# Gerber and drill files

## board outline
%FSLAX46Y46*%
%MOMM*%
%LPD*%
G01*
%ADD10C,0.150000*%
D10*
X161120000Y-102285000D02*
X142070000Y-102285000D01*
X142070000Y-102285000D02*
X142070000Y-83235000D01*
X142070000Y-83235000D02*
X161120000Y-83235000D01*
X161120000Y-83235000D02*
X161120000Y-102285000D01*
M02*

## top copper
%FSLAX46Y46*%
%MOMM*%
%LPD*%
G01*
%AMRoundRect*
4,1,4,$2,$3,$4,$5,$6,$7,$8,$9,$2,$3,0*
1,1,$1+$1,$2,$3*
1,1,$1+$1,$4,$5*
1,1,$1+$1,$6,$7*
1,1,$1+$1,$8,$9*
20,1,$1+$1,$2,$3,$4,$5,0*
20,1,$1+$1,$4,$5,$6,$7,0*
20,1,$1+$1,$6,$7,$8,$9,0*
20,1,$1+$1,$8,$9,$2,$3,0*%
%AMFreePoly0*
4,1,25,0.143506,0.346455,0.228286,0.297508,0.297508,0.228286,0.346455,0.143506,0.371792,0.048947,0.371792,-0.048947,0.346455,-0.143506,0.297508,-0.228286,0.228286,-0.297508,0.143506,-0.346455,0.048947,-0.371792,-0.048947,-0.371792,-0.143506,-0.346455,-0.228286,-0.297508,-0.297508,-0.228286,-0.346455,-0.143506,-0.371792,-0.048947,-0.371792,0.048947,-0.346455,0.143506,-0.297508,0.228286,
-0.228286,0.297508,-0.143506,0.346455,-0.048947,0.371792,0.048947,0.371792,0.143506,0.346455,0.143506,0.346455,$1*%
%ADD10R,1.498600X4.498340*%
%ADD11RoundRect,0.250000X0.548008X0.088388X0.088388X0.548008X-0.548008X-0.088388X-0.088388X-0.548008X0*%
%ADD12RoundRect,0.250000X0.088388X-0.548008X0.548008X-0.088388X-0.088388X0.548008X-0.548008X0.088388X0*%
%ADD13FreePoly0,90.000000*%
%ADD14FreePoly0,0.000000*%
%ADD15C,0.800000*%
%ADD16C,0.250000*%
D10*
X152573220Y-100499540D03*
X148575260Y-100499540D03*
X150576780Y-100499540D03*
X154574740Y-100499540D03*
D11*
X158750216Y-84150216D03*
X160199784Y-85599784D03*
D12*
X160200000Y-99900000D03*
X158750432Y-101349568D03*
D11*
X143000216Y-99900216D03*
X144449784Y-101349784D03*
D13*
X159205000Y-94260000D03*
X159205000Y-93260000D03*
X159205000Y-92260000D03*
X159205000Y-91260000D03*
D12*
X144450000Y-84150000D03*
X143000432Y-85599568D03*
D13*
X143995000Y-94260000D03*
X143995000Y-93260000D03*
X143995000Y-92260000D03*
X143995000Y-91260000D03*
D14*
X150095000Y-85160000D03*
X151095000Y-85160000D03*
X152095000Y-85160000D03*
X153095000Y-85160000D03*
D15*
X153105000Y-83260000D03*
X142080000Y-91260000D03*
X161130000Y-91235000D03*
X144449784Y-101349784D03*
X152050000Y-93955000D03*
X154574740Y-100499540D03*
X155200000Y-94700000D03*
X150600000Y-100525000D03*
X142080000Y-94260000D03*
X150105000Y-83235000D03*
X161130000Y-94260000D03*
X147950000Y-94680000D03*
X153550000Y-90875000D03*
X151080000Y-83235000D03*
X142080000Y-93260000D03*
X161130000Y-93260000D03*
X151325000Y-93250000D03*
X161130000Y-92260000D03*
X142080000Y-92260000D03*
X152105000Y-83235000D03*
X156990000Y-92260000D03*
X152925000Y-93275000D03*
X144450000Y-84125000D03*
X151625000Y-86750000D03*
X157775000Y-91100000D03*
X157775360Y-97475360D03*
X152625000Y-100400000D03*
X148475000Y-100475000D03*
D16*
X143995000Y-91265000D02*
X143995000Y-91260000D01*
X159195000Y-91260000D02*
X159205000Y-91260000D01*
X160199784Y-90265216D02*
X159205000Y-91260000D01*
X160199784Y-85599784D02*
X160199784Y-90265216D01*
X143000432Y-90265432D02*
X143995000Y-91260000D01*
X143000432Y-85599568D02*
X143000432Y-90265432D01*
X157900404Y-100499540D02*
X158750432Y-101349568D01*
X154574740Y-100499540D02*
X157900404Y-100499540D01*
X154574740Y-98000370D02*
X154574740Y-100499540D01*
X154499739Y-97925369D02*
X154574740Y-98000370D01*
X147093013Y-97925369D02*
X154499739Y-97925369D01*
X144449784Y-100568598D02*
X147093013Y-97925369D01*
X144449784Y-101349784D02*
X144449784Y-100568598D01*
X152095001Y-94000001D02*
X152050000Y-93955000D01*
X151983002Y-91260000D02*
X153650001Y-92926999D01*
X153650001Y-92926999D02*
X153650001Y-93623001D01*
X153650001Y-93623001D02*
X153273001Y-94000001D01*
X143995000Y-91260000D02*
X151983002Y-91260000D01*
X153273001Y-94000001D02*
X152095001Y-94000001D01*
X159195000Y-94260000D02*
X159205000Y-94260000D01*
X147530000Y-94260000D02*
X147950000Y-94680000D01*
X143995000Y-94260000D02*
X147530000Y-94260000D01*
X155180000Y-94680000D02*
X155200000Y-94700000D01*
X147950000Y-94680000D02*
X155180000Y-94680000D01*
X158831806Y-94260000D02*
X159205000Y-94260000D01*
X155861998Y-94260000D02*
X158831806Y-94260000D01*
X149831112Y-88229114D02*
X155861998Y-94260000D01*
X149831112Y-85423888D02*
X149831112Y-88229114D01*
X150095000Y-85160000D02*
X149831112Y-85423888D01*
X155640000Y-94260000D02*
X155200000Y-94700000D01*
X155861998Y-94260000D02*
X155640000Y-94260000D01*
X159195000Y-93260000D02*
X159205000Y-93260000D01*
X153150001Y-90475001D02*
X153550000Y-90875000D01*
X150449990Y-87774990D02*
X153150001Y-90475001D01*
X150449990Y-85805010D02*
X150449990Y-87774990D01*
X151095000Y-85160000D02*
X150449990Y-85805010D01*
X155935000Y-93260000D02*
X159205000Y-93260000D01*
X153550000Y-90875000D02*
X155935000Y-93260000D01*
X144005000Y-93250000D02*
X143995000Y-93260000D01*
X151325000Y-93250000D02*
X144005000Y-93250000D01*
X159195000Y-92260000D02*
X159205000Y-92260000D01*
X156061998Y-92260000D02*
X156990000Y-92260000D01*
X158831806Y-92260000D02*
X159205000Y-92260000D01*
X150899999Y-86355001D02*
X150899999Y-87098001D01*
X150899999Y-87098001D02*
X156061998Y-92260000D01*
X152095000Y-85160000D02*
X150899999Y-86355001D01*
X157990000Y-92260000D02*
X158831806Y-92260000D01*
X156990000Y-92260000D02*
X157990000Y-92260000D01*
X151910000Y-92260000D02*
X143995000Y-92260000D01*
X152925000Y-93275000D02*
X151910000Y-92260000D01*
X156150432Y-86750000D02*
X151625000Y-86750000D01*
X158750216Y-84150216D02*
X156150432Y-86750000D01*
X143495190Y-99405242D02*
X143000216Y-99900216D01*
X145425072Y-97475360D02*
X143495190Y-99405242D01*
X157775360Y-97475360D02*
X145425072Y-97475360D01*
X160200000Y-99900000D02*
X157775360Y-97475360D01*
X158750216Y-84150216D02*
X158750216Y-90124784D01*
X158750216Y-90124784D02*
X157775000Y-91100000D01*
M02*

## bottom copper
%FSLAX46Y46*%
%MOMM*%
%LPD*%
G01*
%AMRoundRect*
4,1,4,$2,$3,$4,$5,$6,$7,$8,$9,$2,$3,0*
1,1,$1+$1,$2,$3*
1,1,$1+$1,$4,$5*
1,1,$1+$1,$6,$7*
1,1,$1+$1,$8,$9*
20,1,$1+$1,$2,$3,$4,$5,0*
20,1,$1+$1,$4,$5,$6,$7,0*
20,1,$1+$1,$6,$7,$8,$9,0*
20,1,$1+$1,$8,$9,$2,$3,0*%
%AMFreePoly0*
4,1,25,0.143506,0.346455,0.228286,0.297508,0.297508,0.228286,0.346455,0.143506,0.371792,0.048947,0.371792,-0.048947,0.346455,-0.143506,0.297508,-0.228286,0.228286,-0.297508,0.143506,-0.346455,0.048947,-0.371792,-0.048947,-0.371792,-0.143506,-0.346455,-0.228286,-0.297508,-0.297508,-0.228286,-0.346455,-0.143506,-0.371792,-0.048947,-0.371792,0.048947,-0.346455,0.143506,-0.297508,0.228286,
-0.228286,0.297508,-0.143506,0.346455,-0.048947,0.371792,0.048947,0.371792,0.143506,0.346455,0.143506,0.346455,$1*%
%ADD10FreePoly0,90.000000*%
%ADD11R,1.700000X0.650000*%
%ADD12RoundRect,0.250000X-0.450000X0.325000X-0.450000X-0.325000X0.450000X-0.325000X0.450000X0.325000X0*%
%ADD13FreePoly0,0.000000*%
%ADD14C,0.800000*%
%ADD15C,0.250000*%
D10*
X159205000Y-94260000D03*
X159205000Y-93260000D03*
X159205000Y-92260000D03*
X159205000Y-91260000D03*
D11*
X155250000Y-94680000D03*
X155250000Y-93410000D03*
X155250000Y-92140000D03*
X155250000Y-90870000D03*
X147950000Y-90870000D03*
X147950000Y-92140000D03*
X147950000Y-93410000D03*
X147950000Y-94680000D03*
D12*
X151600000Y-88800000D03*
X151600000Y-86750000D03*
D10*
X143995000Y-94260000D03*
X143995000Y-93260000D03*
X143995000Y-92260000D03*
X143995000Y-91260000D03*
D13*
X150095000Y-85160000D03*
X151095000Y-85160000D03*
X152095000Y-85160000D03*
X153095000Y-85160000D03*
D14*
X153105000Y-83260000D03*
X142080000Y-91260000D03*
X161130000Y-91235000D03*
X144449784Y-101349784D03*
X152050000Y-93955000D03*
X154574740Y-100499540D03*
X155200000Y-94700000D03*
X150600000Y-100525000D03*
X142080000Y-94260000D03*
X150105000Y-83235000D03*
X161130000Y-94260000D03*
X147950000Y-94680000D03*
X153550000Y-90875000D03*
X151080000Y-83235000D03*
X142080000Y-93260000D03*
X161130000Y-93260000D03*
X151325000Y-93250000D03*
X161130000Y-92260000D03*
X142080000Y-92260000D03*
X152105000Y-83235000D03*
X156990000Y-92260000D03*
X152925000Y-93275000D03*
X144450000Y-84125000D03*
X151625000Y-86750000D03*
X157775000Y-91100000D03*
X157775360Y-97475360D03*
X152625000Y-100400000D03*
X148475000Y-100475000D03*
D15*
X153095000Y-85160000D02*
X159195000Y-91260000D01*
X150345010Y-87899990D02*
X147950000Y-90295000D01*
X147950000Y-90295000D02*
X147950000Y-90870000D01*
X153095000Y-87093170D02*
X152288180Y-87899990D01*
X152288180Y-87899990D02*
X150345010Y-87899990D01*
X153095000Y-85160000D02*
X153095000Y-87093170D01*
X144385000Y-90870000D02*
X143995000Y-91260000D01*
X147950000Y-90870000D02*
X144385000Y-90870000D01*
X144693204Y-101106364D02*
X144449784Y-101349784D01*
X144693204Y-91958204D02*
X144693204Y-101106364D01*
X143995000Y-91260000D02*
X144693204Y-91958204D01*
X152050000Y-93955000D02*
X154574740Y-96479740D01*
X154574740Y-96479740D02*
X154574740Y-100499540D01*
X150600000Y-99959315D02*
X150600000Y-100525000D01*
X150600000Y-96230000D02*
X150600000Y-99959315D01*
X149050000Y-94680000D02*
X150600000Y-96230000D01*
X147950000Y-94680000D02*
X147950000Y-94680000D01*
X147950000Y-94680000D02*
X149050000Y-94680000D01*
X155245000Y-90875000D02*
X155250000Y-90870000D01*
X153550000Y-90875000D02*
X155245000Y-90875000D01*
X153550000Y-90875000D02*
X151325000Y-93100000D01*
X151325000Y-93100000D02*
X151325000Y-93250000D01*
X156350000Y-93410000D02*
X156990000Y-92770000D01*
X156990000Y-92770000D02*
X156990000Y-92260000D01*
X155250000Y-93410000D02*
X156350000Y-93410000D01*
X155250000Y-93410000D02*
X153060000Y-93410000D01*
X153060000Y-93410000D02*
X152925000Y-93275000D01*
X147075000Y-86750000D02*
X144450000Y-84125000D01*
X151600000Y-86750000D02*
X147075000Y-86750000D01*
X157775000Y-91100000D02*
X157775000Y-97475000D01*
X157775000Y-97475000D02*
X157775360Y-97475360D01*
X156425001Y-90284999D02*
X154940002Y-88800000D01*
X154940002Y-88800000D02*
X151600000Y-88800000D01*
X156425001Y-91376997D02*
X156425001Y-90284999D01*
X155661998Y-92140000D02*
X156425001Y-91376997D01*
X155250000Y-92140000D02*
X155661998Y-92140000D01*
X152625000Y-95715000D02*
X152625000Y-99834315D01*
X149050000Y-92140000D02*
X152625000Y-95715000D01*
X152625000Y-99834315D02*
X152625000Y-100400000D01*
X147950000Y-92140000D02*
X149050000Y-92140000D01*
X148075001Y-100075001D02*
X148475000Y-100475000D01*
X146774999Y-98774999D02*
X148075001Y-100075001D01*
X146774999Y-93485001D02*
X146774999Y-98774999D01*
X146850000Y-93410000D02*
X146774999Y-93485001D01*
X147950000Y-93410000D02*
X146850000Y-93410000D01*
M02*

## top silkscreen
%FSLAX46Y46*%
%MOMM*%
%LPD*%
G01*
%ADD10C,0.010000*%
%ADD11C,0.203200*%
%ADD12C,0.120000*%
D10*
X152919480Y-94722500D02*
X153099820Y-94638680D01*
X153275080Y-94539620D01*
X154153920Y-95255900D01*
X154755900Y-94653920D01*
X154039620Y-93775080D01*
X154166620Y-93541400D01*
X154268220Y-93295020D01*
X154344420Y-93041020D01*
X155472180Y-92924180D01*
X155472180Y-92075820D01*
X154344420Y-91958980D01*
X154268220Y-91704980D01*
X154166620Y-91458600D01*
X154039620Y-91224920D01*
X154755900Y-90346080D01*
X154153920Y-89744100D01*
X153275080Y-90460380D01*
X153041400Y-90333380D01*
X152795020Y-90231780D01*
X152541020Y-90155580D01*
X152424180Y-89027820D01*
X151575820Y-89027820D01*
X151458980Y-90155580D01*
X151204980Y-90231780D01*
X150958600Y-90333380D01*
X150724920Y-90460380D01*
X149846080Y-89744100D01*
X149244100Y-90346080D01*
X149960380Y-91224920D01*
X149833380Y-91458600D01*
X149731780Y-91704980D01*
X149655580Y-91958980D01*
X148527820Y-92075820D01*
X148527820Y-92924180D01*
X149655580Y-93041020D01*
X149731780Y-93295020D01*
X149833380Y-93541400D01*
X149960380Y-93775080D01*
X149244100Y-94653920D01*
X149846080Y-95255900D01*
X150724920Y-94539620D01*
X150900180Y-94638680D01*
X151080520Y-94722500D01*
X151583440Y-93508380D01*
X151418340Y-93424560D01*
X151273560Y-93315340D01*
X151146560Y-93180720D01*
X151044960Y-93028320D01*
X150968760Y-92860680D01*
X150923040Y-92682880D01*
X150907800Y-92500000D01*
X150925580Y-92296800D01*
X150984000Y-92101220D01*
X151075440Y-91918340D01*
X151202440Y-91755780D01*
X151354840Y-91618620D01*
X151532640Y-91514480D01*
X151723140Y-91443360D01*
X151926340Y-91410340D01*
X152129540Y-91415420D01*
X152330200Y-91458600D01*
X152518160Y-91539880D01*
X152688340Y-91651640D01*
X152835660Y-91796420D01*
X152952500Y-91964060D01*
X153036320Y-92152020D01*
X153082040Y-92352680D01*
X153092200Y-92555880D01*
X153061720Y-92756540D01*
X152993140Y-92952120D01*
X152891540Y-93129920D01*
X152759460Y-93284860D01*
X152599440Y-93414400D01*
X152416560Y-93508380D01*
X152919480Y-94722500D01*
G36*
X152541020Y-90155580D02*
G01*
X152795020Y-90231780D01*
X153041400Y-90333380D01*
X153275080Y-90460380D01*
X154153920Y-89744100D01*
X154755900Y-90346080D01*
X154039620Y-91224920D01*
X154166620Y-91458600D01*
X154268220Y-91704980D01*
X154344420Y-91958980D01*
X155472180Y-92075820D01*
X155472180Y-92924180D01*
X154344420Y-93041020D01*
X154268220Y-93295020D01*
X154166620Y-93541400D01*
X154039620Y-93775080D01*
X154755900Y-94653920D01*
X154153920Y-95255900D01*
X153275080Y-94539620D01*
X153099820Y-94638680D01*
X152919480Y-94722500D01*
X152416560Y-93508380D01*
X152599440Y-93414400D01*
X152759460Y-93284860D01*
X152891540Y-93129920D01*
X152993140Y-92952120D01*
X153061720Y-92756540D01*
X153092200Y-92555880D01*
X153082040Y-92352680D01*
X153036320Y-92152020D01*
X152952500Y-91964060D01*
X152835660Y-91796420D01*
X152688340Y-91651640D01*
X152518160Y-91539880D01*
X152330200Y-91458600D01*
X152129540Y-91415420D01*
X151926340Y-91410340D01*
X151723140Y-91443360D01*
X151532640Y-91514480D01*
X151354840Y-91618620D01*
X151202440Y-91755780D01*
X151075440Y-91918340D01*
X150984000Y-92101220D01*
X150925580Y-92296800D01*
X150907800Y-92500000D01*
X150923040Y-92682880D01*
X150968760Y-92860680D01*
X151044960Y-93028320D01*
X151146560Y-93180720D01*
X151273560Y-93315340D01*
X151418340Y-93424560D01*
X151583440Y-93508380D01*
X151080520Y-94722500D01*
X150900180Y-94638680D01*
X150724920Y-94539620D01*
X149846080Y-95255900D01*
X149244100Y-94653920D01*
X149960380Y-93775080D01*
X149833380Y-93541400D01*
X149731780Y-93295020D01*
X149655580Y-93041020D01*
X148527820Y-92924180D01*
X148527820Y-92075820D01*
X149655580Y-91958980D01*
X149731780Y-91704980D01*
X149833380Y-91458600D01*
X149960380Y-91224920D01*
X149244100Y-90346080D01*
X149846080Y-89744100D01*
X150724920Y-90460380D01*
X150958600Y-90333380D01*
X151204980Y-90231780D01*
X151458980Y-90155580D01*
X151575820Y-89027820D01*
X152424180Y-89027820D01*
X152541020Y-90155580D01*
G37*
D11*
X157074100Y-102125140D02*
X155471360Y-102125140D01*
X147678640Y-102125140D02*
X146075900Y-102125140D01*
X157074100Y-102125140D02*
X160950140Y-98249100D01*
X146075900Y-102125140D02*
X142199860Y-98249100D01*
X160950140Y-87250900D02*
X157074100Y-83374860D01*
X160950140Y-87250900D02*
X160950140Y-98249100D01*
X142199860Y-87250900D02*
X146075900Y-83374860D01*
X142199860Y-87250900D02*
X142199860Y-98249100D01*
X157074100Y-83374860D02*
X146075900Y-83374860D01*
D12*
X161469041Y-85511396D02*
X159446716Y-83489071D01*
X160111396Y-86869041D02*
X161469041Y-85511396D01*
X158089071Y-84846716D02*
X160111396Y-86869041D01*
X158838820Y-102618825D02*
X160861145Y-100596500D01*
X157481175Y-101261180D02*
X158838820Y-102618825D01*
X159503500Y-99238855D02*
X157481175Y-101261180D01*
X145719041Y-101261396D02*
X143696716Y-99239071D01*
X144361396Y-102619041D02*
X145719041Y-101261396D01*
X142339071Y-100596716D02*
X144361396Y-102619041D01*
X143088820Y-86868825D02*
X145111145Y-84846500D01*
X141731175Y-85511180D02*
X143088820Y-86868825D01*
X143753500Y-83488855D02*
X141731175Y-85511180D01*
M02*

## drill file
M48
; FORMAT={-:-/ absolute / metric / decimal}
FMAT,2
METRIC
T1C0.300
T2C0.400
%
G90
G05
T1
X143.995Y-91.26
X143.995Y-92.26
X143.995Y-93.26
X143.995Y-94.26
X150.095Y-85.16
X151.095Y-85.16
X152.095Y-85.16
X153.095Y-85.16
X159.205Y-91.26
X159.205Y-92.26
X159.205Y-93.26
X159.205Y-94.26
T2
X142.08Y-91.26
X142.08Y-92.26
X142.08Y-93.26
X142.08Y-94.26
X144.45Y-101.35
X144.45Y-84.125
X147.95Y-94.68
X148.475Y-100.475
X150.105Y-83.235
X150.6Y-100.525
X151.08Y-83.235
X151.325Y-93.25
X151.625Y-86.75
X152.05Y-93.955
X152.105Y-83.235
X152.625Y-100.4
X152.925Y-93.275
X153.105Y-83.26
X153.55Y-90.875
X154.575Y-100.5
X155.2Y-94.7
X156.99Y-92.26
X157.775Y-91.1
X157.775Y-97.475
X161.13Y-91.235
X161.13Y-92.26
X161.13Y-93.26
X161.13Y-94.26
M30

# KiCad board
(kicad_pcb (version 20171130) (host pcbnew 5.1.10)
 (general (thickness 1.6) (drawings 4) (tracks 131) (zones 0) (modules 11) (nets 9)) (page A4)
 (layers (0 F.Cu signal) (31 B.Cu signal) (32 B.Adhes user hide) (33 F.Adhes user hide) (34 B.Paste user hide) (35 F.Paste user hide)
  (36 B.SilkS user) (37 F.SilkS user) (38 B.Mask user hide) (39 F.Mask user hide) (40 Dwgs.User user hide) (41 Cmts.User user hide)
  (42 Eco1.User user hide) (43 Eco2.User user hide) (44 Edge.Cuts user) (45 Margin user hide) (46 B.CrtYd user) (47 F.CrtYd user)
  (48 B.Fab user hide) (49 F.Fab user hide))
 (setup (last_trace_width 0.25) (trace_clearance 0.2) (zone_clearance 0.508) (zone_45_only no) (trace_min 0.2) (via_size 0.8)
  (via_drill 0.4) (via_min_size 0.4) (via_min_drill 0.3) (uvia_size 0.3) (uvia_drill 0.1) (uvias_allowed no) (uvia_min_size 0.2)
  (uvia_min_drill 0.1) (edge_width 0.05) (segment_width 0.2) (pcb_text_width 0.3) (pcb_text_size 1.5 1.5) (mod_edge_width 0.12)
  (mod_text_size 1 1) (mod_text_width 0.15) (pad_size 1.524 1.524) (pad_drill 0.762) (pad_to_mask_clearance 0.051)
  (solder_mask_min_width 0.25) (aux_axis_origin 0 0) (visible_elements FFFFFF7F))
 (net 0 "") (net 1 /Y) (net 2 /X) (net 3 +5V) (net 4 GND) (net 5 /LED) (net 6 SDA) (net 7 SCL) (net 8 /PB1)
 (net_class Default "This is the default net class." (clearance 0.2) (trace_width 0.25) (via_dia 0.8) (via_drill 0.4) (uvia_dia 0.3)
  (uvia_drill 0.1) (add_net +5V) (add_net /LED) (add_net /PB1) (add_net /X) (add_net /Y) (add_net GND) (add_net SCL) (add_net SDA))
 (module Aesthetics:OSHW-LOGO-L (layer F.Cu) (at 152 92.5)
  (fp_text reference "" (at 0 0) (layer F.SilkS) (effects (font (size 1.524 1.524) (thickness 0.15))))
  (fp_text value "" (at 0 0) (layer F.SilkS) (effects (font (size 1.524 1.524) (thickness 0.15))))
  (fp_poly
   (pts (xy 0.91948 2.2225) (xy 1.09982 2.13868) (xy 1.27508 2.03962) (xy 2.15392 2.7559) (xy 2.7559 2.15392) (xy 2.03962 1.27508)
    (xy 2.16662 1.0414) (xy 2.26822 0.79502) (xy 2.34442 0.54102) (xy 3.47218 0.42418) (xy 3.47218 -0.42418) (xy 2.34442 -0.54102)
    (xy 2.26822 -0.79502) (xy 2.16662 -1.0414) (xy 2.03962 -1.27508) (xy 2.7559 -2.15392) (xy 2.15392 -2.7559) (xy 1.27508 -2.03962)
    (xy 1.0414 -2.16662) (xy 0.79502 -2.26822) (xy 0.54102 -2.34442) (xy 0.42418 -3.47218) (xy -0.42418 -3.47218) (xy -0.54102 -2.34442)
    (xy -0.79502 -2.26822) (xy -1.0414 -2.16662) (xy -1.27508 -2.03962) (xy -2.15392 -2.7559) (xy -2.7559 -2.15392) (xy -2.03962 -1.27508)
    (xy -2.16662 -1.0414) (xy -2.26822 -0.79502) (xy -2.34442 -0.54102) (xy -3.47218 -0.42418) (xy -3.47218 0.42418) (xy -2.34442 0.54102)
    (xy -2.26822 0.79502) (xy -2.16662 1.0414) (xy -2.03962 1.27508) (xy -2.7559 2.15392) (xy -2.15392 2.7559) (xy -1.27508 2.03962)
    (xy -1.09982 2.13868) (xy -0.91948 2.2225) (xy -0.41656 1.00838) (xy -0.58166 0.92456) (xy -0.72644 0.81534) (xy -0.85344 0.68072)
    (xy -0.95504 0.52832) (xy -1.03124 0.36068) (xy -1.07696 0.18288) (xy -1.0922 0) (xy -1.07442 -0.2032) (xy -1.016 -0.39878)
    (xy -0.92456 -0.58166) (xy -0.79756 -0.74422) (xy -0.64516 -0.88138) (xy -0.46736 -0.98552) (xy -0.27686 -1.05664)
    (xy -0.07366 -1.08966) (xy 0.12954 -1.08458) (xy 0.3302 -1.0414) (xy 0.51816 -0.96012) (xy 0.68834 -0.84836) (xy 0.83566 -0.70358)
    (xy 0.9525 -0.53594) (xy 1.03632 -0.34798) (xy 1.08204 -0.14732) (xy 1.0922 0.05588) (xy 1.06172 0.25654) (xy 0.99314 0.45212)
    (xy 0.89154 0.62992) (xy 0.75946 0.78486) (xy 0.59944 0.9144) (xy 0.41656 1.00838))
   (layer F.SilkS) (width 0.01)))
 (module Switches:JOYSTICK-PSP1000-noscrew (layer F.Cu) (at 151.575 92.75 180)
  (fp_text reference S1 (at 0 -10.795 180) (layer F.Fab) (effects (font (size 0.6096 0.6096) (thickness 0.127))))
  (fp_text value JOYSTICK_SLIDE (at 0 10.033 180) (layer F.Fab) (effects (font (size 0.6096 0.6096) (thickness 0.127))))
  (fp_line (start -5.4991 -9.37514) (end -3.89636 -9.37514) (layer F.SilkS) (width 0.2032))
  (fp_line (start 3.89636 -9.37514) (end 5.4991 -9.37514) (layer F.SilkS) (width 0.2032))
  (fp_line (start -5.4991 -9.37514) (end -9.37514 -5.4991) (layer F.SilkS) (width 0.2032))
  (fp_line (start 5.4991 -9.37514) (end 9.37514 -5.4991) (layer F.SilkS) (width 0.2032))
  (fp_line (start -9.37514 5.4991) (end -5.4991 9.37514) (layer F.SilkS) (width 0.2032))
  (fp_line (start -9.37514 5.4991) (end -9.37514 -5.4991) (layer F.SilkS) (width 0.2032))
  (fp_line (start 9.37514 5.4991) (end 5.4991 9.37514) (layer F.SilkS) (width 0.2032))
  (fp_line (start 9.37514 5.4991) (end 9.37514 -5.4991) (layer F.SilkS) (width 0.2032))
  (fp_line (start -5.4991 9.37514) (end 5.4991 9.37514) (layer F.SilkS) (width 0.2032))
  (pad Y smd rect (at -0.99822 -7.74954 270) (size 4.49834 1.4986) (layers F.Cu F.Paste F.Mask) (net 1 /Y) (solder_mask_margin 0.1016))
  (pad X smd rect (at 2.99974 -7.74954 270) (size 4.49834 1.4986) (layers F.Cu F.Paste F.Mask) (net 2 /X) (solder_mask_margin 0.1016))
  (pad VCC smd rect (at 0.99822 -7.74954 270) (size 4.49834 1.4986) (layers F.Cu F.Paste F.Mask) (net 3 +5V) (solder_mask_margin 0.1016))
  (pad GND smd rect (at -2.99974 -7.74954 270) (size 4.49834 1.4986) (layers F.Cu F.Paste F.Mask) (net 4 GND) (solder_mask_margin 0.1016)))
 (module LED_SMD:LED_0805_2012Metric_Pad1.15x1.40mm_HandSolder (layer F.Cu) (at 159.475 84.875 135)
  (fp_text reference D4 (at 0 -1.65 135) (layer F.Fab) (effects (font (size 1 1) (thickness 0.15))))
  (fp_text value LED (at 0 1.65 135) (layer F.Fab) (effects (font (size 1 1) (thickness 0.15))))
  (fp_line (start -1.86 0.96) (end 1 0.96) (layer F.SilkS) (width 0.12))
  (fp_line (start -1.86 -0.96) (end -1.86 0.96) (layer F.SilkS) (width 0.12))
  (fp_line (start 1 -0.96) (end -1.86 -0.96) (layer F.SilkS) (width 0.12))
  (pad 2 smd roundrect (at 1.025 0 135) (size 1.15 1.4) (layers F.Cu F.Paste F.Mask) (roundrect_rratio 0.217391) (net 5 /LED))
  (pad 1 smd roundrect (at -1.025 0 135) (size 1.15 1.4) (layers F.Cu F.Paste F.Mask) (roundrect_rratio 0.217391) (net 4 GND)))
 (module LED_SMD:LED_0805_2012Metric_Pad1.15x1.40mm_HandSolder (layer F.Cu) (at 159.475216 100.624784 45)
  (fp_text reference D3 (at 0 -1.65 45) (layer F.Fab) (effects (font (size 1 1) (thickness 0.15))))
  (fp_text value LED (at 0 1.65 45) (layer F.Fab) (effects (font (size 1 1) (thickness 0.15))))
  (fp_line (start -1.86 0.96) (end 1 0.96) (layer F.SilkS) (width 0.12))
  (fp_line (start -1.86 -0.96) (end -1.86 0.96) (layer F.SilkS) (width 0.12))
  (fp_line (start 1 -0.96) (end -1.86 -0.96) (layer F.SilkS) (width 0.12))
  (pad 2 smd roundrect (at 1.025 0 45) (size 1.15 1.4) (layers F.Cu F.Paste F.Mask) (roundrect_rratio 0.217391) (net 5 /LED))
  (pad 1 smd roundrect (at -1.025 0 45) (size 1.15 1.4) (layers F.Cu F.Paste F.Mask) (roundrect_rratio 0.217391) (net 4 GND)))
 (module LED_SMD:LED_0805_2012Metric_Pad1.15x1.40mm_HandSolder (layer F.Cu) (at 143.725 100.625 135)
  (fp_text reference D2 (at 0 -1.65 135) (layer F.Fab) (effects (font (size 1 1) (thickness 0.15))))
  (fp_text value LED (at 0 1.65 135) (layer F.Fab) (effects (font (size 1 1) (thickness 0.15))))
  (fp_line (start -1.86 0.96) (end 1 0.96) (layer F.SilkS) (width 0.12))
  (fp_line (start -1.86 -0.96) (end -1.86 0.96) (layer F.SilkS) (width 0.12))
  (fp_line (start 1 -0.96) (end -1.86 -0.96) (layer F.SilkS) (width 0.12))
  (pad 2 smd roundrect (at 1.025 0 135) (size 1.15 1.4) (layers F.Cu F.Paste F.Mask) (roundrect_rratio 0.217391) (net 5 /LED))
  (pad 1 smd roundrect (at -1.025 0 135) (size 1.15 1.4) (layers F.Cu F.Paste F.Mask) (roundrect_rratio 0.217391) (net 4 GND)))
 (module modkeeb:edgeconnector (layer F.Cu) (at 161.205 92.76 90)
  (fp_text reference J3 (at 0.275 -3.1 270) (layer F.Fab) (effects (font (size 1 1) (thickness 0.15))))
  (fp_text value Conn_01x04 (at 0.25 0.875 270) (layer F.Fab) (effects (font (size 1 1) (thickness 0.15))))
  (pad 1 thru_hole custom (at -1.5 -2 90) (size 0.75 0.75) (drill 0.3) (layers *.Cu *.Mask) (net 3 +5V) (zone_connect 0)
   (options (clearance outline) (anchor circle)) (primitives))
  (pad 2 thru_hole custom (at -0.5 -2 90) (size 0.75 0.75) (drill 0.3) (layers *.Cu *.Mask) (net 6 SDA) (zone_connect 0)
   (options (clearance outline) (anchor circle)) (primitives))
  (pad 3 thru_hole custom (at 0.5 -2 90) (size 0.75 0.75) (drill 0.3) (layers *.Cu *.Mask) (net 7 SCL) (zone_connect 0)
   (options (clearance outline) (anchor circle)) (primitives))
  (pad 4 thru_hole custom (at 1.5 -2 90) (size 0.75 0.75) (drill 0.3) (layers *.Cu *.Mask) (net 4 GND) (zone_connect 0)
   (options (clearance outline) (anchor circle)) (primitives)))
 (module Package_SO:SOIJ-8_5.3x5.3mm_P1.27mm (layer B.Cu) (at 151.6 92.775)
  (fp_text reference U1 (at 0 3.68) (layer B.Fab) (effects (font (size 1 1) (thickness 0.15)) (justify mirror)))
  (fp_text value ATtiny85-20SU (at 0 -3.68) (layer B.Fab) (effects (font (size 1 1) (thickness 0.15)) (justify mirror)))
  (pad 8 smd rect (at 3.65 1.905) (size 1.7 0.65) (layers B.Cu B.Paste B.Mask) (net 3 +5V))
  (pad 7 smd rect (at 3.65 0.635) (size 1.7 0.65) (layers B.Cu B.Paste B.Mask) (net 7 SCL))
  (pad 6 smd rect (at 3.65 -0.635) (size 1.7 0.65) (layers B.Cu B.Paste B.Mask) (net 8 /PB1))
  (pad 5 smd rect (at 3.65 -1.905) (size 1.7 0.65) (layers B.Cu B.Paste B.Mask) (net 6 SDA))
  (pad 4 smd rect (at -3.65 -1.905) (size 1.7 0.65) (layers B.Cu B.Paste B.Mask) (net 4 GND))
  (pad 3 smd rect (at -3.65 -0.635) (size 1.7 0.65) (layers B.Cu B.Paste B.Mask) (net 1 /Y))
  (pad 2 smd rect (at -3.65 0.635) (size 1.7 0.65) (layers B.Cu B.Paste B.Mask) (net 2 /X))
  (pad 1 smd rect (at -3.65 1.905) (size 1.7 0.65) (layers B.Cu B.Paste B.Mask) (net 3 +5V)))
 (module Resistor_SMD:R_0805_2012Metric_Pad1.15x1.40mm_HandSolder (layer B.Cu) (at 151.6 87.775 270)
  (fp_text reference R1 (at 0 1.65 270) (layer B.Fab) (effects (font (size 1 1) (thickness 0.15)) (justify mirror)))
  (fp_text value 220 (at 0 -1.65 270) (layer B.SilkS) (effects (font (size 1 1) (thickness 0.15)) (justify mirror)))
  (pad 2 smd roundrect (at 1.025 0 270) (size 1.15 1.4) (layers B.Cu B.Paste B.Mask) (roundrect_rratio 0.217391) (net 8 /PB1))
  (pad 1 smd roundrect (at -1.025 0 270) (size 1.15 1.4) (layers B.Cu B.Paste B.Mask) (roundrect_rratio 0.217391) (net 5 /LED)))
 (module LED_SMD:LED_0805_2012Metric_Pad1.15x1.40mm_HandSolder (layer F.Cu) (at 143.725216 84.874784 45)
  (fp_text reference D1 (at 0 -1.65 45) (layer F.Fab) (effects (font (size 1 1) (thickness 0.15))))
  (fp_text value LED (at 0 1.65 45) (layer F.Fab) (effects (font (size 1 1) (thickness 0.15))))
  (fp_line (start -1.86 0.96) (end 1 0.96) (layer F.SilkS) (width 0.12))
  (fp_line (start -1.86 -0.96) (end -1.86 0.96) (layer F.SilkS) (width 0.12))
  (fp_line (start 1 -0.96) (end -1.86 -0.96) (layer F.SilkS) (width 0.12))
  (pad 2 smd roundrect (at 1.025 0 45) (size 1.15 1.4) (layers F.Cu F.Paste F.Mask) (roundrect_rratio 0.217391) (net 5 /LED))
  (pad 1 smd roundrect (at -1.025 0 45) (size 1.15 1.4) (layers F.Cu F.Paste F.Mask) (roundrect_rratio 0.217391) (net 4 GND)))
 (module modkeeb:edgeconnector (layer B.Cu) (at 141.995 92.76 90)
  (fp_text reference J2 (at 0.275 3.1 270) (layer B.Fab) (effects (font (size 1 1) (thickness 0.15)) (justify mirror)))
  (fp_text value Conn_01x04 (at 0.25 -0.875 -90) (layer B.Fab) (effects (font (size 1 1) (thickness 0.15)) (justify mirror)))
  (pad 1 thru_hole custom (at -1.5 2 90) (size 0.75 0.75) (drill 0.3) (layers *.Cu *.Mask) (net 3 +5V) (zone_connect 0)
   (options (clearance outline) (anchor circle)) (primitives))
  (pad 2 thru_hole custom (at -0.5 2 90) (size 0.75 0.75) (drill 0.3) (layers *.Cu *.Mask) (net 6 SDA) (zone_connect 0)
   (options (clearance outline) (anchor circle)) (primitives))
  (pad 3 thru_hole custom (at 0.5 2 90) (size 0.75 0.75) (drill 0.3) (layers *.Cu *.Mask) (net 7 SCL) (zone_connect 0)
   (options (clearance outline) (anchor circle)) (primitives))
  (pad 4 thru_hole custom (at 1.5 2 90) (size 0.75 0.75) (drill 0.3) (layers *.Cu *.Mask) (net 4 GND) (zone_connect 0)
   (options (clearance outline) (anchor circle)) (primitives)))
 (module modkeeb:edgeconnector (layer B.Cu) (at 151.595 83.16)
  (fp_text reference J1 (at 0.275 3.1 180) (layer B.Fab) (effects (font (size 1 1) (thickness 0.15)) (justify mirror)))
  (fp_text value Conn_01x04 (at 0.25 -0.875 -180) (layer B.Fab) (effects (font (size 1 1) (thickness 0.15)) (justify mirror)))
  (pad 1 thru_hole custom (at -1.5 2) (size 0.75 0.75) (drill 0.3) (layers *.Cu *.Mask) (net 3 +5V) (zone_connect 0)
   (options (clearance outline) (anchor circle)) (primitives))
  (pad 2 thru_hole custom (at -0.5 2) (size 0.75 0.75) (drill 0.3) (layers *.Cu *.Mask) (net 6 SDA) (zone_connect 0)
   (options (clearance outline) (anchor circle)) (primitives))
  (pad 3 thru_hole custom (at 0.5 2) (size 0.75 0.75) (drill 0.3) (layers *.Cu *.Mask) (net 7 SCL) (zone_connect 0)
   (options (clearance outline) (anchor circle)) (primitives))
  (pad 4 thru_hole custom (at 1.5 2) (size 0.75 0.75) (drill 0.3) (layers *.Cu *.Mask) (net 4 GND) (zone_connect 0)
   (options (clearance outline) (anchor circle)) (primitives)))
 (gr_line (start 161.12 102.285) (end 142.07 102.285) (layer Edge.Cuts) (width 0.15))
 (gr_line (start 142.07 102.285) (end 142.07 83.235) (layer Edge.Cuts) (width 0.15))
 (gr_line (start 142.07 83.235) (end 161.12 83.235) (layer Edge.Cuts) (width 0.15))
 (gr_line (start 161.12 83.235) (end 161.12 102.285) (layer Edge.Cuts) (width 0.15))
 (via (at 153.105 83.26) (size 0.8) (drill 0.4) (layers F.Cu B.Cu) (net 4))
 (segment (start 143.995 91.265) (end 143.995 91.26) (width 0.25) (layer F.Cu) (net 4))
 (via (at 142.08 91.26) (size 0.8) (drill 0.4) (layers F.Cu B.Cu) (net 4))
 (via (at 161.13 91.235) (size 0.8) (drill 0.4) (layers F.Cu B.Cu) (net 4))
 (segment (start 159.195 91.26) (end 159.205 91.26) (width 0.25) (layer F.Cu) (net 4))
 (segment (start 153.095 85.16) (end 159.195 91.26) (width 0.25) (layer B.Cu) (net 4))
 (segment (start 160.199784 90.265216) (end 159.205 91.26) (width 0.25) (layer F.Cu) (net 4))
 (segment (start 160.199784 85.599784) (end 160.199784 90.265216) (width 0.25) (layer F.Cu) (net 4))
 (segment (start 150.34501 87.89999) (end 147.95 90.295) (width 0.25) (layer B.Cu) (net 4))
 (segment (start 147.95 90.295) (end 147.95 90.87) (width 0.25) (layer B.Cu) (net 4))
 (segment (start 153.095 87.09317) (end 152.28818 87.89999) (width 0.25) (layer B.Cu) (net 4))
 (segment (start 152.28818 87.89999) (end 150.34501 87.89999) (width 0.25) (layer B.Cu) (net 4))
 (segment (start 153.095 85.16) (end 153.095 87.09317) (width 0.25) (layer B.Cu) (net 4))
 (segment (start 144.385 90.87) (end 143.995 91.26) (width 0.25) (layer B.Cu) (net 4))
 (segment (start 147.95 90.87) (end 144.385 90.87) (width 0.25) (layer B.Cu) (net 4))
 (segment (start 143.000432 90.265432) (end 143.995 91.26) (width 0.25) (layer F.Cu) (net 4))
 (segment (start 143.000432 85.599568) (end 143.000432 90.265432) (width 0.25) (layer F.Cu) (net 4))
 (segment (start 157.900404 100.49954) (end 158.750432 101.349568) (width 0.25) (layer F.Cu) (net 4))
 (segment (start 154.57474 100.49954) (end 157.900404 100.49954) (width 0.25) (layer F.Cu) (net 4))
 (segment (start 154.57474 98.00037) (end 154.57474 100.49954) (width 0.25) (layer F.Cu) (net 4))
 (segment (start 154.499739 97.925369) (end 154.57474 98.00037) (width 0.25) (layer F.Cu) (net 4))
 (segment (start 147.093013 97.925369) (end 154.499739 97.925369) (width 0.25) (layer F.Cu) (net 4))
 (segment (start 144.449784 100.568598) (end 147.093013 97.925369) (width 0.25) (layer F.Cu) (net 4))
 (segment (start 144.449784 101.349784) (end 144.449784 100.568598) (width 0.25) (layer F.Cu) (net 4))
 (via (at 144.449784 101.349784) (size 0.8) (drill 0.4) (layers F.Cu B.Cu) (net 4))
 (segment (start 144.693204 101.106364) (end 144.449784 101.349784) (width 0.25) (layer B.Cu) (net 4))
 (segment (start 144.693204 91.958204) (end 144.693204 101.106364) (width 0.25) (layer B.Cu) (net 4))
 (segment (start 143.995 91.26) (end 144.693204 91.958204) (width 0.25) (layer B.Cu) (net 4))
 (via (at 152.05 93.955) (size 0.8) (drill 0.4) (layers F.Cu B.Cu) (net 4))
 (segment (start 152.095001 94.000001) (end 152.05 93.955) (width 0.25) (layer F.Cu) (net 4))
 (segment (start 151.983002 91.26) (end 153.650001 92.926999) (width 0.25) (layer F.Cu) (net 4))
 (segment (start 153.650001 92.926999) (end 153.650001 93.623001) (width 0.25) (layer F.Cu) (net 4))
 (segment (start 153.650001 93.623001) (end 153.273001 94.000001) (width 0.25) (layer F.Cu) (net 4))
 (segment (start 143.995 91.26) (end 151.983002 91.26) (width 0.25) (layer F.Cu) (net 4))
 (segment (start 153.273001 94.000001) (end 152.095001 94.000001) (width 0.25) (layer F.Cu) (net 4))
 (segment (start 152.05 93.955) (end 154.57474 96.47974) (width 0.25) (layer B.Cu) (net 4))
 (via (at 154.57474 100.49954) (size 0.8) (drill 0.4) (layers F.Cu B.Cu) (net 4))
 (segment (start 154.57474 96.47974) (end 154.57474 100.49954) (width 0.25) (layer B.Cu) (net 4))
 (via (at 155.2 94.7) (size 0.8) (drill 0.4) (layers F.Cu B.Cu) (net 3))
 (via (at 150.6 100.525) (size 0.8) (drill 0.4) (layers F.Cu B.Cu) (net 3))
 (via (at 142.08 94.26) (size 0.8) (drill 0.4) (layers F.Cu B.Cu) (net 3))
 (segment (start 159.195 94.26) (end 159.205 94.26) (width 0.25) (layer F.Cu) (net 3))
 (via (at 150.105 83.235) (size 0.8) (drill 0.4) (layers F.Cu B.Cu) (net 3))
 (via (at 161.13 94.26) (size 0.8) (drill 0.4) (layers F.Cu B.Cu) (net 3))
 (segment (start 150.6 99.959315) (end 150.6 100.525) (width 0.25) (layer B.Cu) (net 3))
 (segment (start 150.6 96.23) (end 150.6 99.959315) (width 0.25) (layer B.Cu) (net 3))
 (segment (start 149.05 94.68) (end 150.6 96.23) (width 0.25) (layer B.Cu) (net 3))
 (segment (start 147.95 94.68) (end 147.95 94.68) (width 0.25) (layer B.Cu) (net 3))
 (segment (start 147.95 94.68) (end 149.05 94.68) (width 0.25) (layer B.Cu) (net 3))
 (via (at 147.95 94.68) (size 0.8) (drill 0.4) (layers F.Cu B.Cu) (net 3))
 (segment (start 147.53 94.26) (end 147.95 94.68) (width 0.25) (layer F.Cu) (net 3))
 (segment (start 143.995 94.26) (end 147.53 94.26) (width 0.25) (layer F.Cu) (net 3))
 (segment (start 155.18 94.68) (end 155.2 94.7) (width 0.25) (layer F.Cu) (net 3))
 (segment (start 147.95 94.68) (end 155.18 94.68) (width 0.25) (layer F.Cu) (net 3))
 (segment (start 158.831806 94.26) (end 159.205 94.26) (width 0.25) (layer F.Cu) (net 3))
 (segment (start 155.861998 94.26) (end 158.831806 94.26) (width 0.25) (layer F.Cu) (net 3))
 (segment (start 149.831112 88.229114) (end 155.861998 94.26) (width 0.25) (layer F.Cu) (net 3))
 (segment (start 149.831112 85.423888) (end 149.831112 88.229114) (width 0.25) (layer F.Cu) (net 3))
 (segment (start 150.095 85.16) (end 149.831112 85.423888) (width 0.25) (layer F.Cu) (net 3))
 (segment (start 155.64 94.26) (end 155.2 94.7) (width 0.25) (layer F.Cu) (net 3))
 (segment (start 155.861998 94.26) (end 155.64 94.26) (width 0.25) (layer F.Cu) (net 3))
 (via (at 153.55 90.875) (size 0.8) (drill 0.4) (layers F.Cu B.Cu) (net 6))
 (via (at 151.08 83.235) (size 0.8) (drill 0.4) (layers F.Cu B.Cu) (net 6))
 (via (at 142.08 93.26) (size 0.8) (drill 0.4) (layers F.Cu B.Cu) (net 6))
 (via (at 161.13 93.26) (size 0.8) (drill 0.4) (layers F.Cu B.Cu) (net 6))
 (segment (start 159.195 93.26) (end 159.205 93.26) (width 0.25) (layer F.Cu) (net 6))
 (segment (start 155.245 90.875) (end 155.25 90.87) (width 0.25) (layer B.Cu) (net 6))
 (segment (start 153.55 90.875) (end 155.245 90.875) (width 0.25) (layer B.Cu) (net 6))
 (segment (start 153.150001 90.475001) (end 153.55 90.875) (width 0.25) (layer F.Cu) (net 6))
 (segment (start 150.44999 87.77499) (end 153.150001 90.475001) (width 0.25) (layer F.Cu) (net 6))
 (segment (start 150.44999 85.80501) (end 150.44999 87.77499) (width 0.25) (layer F.Cu) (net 6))
 (segment (start 151.095 85.16) (end 150.44999 85.80501) (width 0.25) (layer F.Cu) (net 6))
 (segment (start 155.935 93.26) (end 159.205 93.26) (width 0.25) (layer F.Cu) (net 6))
 (segment (start 153.55 90.875) (end 155.935 93.26) (width 0.25) (layer F.Cu) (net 6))
 (via (at 151.325 93.25) (size 0.8) (drill 0.4) (layers F.Cu B.Cu) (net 6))
 (segment (start 153.55 90.875) (end 151.325 93.1) (width 0.25) (layer B.Cu) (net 6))
 (segment (start 151.325 93.1) (end 151.325 93.25) (width 0.25) (layer B.Cu) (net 6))
 (segment (start 144.005 93.25) (end 143.995 93.26) (width 0.25) (layer F.Cu) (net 6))
 (segment (start 151.325 93.25) (end 144.005 93.25) (width 0.25) (layer F.Cu) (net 6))
 (via (at 161.13 92.26) (size 0.8) (drill 0.4) (layers F.Cu B.Cu) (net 7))
 (via (at 142.08 92.26) (size 0.8) (drill 0.4) (layers F.Cu B.Cu) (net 7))
 (via (at 152.105 83.235) (size 0.8) (drill 0.4) (layers F.Cu B.Cu) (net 7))
 (segment (start 159.195 92.26) (end 159.205 92.26) (width 0.25) (layer F.Cu) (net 7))
 (segment (start 156.061998 92.26) (end 156.99 92.26) (width 0.25) (layer F.Cu) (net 7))
 (segment (start 158.831806 92.26) (end 159.205 92.26) (width 0.25) (layer F.Cu) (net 7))
 (segment (start 150.899999 86.355001) (end 150.899999 87.098001) (width 0.25) (layer F.Cu) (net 7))
 (segment (start 150.899999 87.098001) (end 156.061998 92.26) (width 0.25) (layer F.Cu) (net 7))
 (segment (start 152.095 85.16) (end 150.899999 86.355001) (width 0.25) (layer F.Cu) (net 7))
 (segment (start 157.99 92.26) (end 158.831806 92.26) (width 0.25) (layer F.Cu) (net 7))
 (segment (start 156.99 92.26) (end 157.99 92.26) (width 0.25) (layer F.Cu) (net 7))
 (via (at 156.99 92.26) (size 0.8) (drill 0.4) (layers F.Cu B.Cu) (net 7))
 (segment (start 156.35 93.41) (end 156.99 92.77) (width 0.25) (layer B.Cu) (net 7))
 (segment (start 156.99 92.77) (end 156.99 92.26) (width 0.25) (layer B.Cu) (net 7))
 (segment (start 155.25 93.41) (end 156.35 93.41) (width 0.25) (layer B.Cu) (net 7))
 (segment (start 155.25 93.41) (end 153.06 93.41) (width 0.25) (layer B.Cu) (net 7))
 (via (at 152.925 93.275) (size 0.8) (drill 0.4) (layers F.Cu B.Cu) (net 7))
 (segment (start 153.06 93.41) (end 152.925 93.275) (width 0.25) (layer B.Cu) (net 7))
 (segment (start 151.91 92.26) (end 143.995 92.26) (width 0.25) (layer F.Cu) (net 7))
 (segment (start 152.925 93.275) (end 151.91 92.26) (width 0.25) (layer F.Cu) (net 7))
 (via (at 144.45 84.125) (size 0.8) (drill 0.4) (layers F.Cu B.Cu) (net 5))
 (via (at 151.625 86.75) (size 0.8) (drill 0.4) (layers F.Cu B.Cu) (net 5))
 (segment (start 156.150432 86.75) (end 151.625 86.75) (width 0.25) (layer F.Cu) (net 5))
 (segment (start 158.750216 84.150216) (end 156.150432 86.75) (width 0.25) (layer F.Cu) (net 5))
 (segment (start 147.075 86.75) (end 144.45 84.125) (width 0.25) (layer B.Cu) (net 5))
 (segment (start 151.6 86.75) (end 147.075 86.75) (width 0.25) (layer B.Cu) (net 5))
 (segment (start 143.49519 99.405242) (end 143.000216 99.900216) (width 0.25) (layer F.Cu) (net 5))
 (segment (start 145.425072 97.47536) (end 143.49519 99.405242) (width 0.25) (layer F.Cu) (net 5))
 (segment (start 157.77536 97.47536) (end 145.425072 97.47536) (width 0.25) (layer F.Cu) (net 5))
 (segment (start 160.2 99.9) (end 157.77536 97.47536) (width 0.25) (layer F.Cu) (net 5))
 (via (at 157.775 91.1) (size 0.8) (drill 0.4) (layers F.Cu B.Cu) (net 5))
 (segment (start 158.750216 84.150216) (end 158.750216 90.124784) (width 0.25) (layer F.Cu) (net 5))
 (segment (start 158.750216 90.124784) (end 157.775 91.1) (width 0.25) (layer F.Cu) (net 5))
 (via (at 157.77536 97.47536) (size 0.8) (drill 0.4) (layers F.Cu B.Cu) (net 5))
 (segment (start 157.775 91.1) (end 157.775 97.475) (width 0.25) (layer B.Cu) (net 5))
 (segment (start 157.775 97.475) (end 157.77536 97.47536) (width 0.25) (layer B.Cu) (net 5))
 (segment (start 156.425001 90.284999) (end 154.940002 88.8) (width 0.25) (layer B.Cu) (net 8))
 (segment (start 154.940002 88.8) (end 151.6 88.8) (width 0.25) (layer B.Cu) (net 8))
 (segment (start 156.425001 91.376997) (end 156.425001 90.284999) (width 0.25) (layer B.Cu) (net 8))
 (segment (start 155.661998 92.14) (end 156.425001 91.376997) (width 0.25) (layer B.Cu) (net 8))
 (segment (start 155.25 92.14) (end 155.661998 92.14) (width 0.25) (layer B.Cu) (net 8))
 (via (at 152.625 100.4) (size 0.8) (drill 0.4) (layers F.Cu B.Cu) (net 1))
 (segment (start 152.625 95.715) (end 152.625 99.834315) (width 0.25) (layer B.Cu) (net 1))
 (segment (start 149.05 92.14) (end 152.625 95.715) (width 0.25) (layer B.Cu) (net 1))
 (segment (start 152.625 99.834315) (end 152.625 100.4) (width 0.25) (layer B.Cu) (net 1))
 (segment (start 147.95 92.14) (end 149.05 92.14) (width 0.25) (layer B.Cu) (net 1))
 (via (at 148.475 100.475) (size 0.8) (drill 0.4) (layers F.Cu B.Cu) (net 2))
 (segment (start 148.075001 100.075001) (end 148.475 100.475) (width 0.25) (layer B.Cu) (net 2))
 (segment (start 146.774999 98.774999) (end 148.075001 100.075001) (width 0.25) (layer B.Cu) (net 2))
 (segment (start 146.774999 93.485001) (end 146.774999 98.774999) (width 0.25) (layer B.Cu) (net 2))
 (segment (start 146.85 93.41) (end 146.774999 93.485001) (width 0.25) (layer B.Cu) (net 2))
 (segment (start 147.95 93.41) (end 146.85 93.41) (width 0.25) (layer B.Cu) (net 2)))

